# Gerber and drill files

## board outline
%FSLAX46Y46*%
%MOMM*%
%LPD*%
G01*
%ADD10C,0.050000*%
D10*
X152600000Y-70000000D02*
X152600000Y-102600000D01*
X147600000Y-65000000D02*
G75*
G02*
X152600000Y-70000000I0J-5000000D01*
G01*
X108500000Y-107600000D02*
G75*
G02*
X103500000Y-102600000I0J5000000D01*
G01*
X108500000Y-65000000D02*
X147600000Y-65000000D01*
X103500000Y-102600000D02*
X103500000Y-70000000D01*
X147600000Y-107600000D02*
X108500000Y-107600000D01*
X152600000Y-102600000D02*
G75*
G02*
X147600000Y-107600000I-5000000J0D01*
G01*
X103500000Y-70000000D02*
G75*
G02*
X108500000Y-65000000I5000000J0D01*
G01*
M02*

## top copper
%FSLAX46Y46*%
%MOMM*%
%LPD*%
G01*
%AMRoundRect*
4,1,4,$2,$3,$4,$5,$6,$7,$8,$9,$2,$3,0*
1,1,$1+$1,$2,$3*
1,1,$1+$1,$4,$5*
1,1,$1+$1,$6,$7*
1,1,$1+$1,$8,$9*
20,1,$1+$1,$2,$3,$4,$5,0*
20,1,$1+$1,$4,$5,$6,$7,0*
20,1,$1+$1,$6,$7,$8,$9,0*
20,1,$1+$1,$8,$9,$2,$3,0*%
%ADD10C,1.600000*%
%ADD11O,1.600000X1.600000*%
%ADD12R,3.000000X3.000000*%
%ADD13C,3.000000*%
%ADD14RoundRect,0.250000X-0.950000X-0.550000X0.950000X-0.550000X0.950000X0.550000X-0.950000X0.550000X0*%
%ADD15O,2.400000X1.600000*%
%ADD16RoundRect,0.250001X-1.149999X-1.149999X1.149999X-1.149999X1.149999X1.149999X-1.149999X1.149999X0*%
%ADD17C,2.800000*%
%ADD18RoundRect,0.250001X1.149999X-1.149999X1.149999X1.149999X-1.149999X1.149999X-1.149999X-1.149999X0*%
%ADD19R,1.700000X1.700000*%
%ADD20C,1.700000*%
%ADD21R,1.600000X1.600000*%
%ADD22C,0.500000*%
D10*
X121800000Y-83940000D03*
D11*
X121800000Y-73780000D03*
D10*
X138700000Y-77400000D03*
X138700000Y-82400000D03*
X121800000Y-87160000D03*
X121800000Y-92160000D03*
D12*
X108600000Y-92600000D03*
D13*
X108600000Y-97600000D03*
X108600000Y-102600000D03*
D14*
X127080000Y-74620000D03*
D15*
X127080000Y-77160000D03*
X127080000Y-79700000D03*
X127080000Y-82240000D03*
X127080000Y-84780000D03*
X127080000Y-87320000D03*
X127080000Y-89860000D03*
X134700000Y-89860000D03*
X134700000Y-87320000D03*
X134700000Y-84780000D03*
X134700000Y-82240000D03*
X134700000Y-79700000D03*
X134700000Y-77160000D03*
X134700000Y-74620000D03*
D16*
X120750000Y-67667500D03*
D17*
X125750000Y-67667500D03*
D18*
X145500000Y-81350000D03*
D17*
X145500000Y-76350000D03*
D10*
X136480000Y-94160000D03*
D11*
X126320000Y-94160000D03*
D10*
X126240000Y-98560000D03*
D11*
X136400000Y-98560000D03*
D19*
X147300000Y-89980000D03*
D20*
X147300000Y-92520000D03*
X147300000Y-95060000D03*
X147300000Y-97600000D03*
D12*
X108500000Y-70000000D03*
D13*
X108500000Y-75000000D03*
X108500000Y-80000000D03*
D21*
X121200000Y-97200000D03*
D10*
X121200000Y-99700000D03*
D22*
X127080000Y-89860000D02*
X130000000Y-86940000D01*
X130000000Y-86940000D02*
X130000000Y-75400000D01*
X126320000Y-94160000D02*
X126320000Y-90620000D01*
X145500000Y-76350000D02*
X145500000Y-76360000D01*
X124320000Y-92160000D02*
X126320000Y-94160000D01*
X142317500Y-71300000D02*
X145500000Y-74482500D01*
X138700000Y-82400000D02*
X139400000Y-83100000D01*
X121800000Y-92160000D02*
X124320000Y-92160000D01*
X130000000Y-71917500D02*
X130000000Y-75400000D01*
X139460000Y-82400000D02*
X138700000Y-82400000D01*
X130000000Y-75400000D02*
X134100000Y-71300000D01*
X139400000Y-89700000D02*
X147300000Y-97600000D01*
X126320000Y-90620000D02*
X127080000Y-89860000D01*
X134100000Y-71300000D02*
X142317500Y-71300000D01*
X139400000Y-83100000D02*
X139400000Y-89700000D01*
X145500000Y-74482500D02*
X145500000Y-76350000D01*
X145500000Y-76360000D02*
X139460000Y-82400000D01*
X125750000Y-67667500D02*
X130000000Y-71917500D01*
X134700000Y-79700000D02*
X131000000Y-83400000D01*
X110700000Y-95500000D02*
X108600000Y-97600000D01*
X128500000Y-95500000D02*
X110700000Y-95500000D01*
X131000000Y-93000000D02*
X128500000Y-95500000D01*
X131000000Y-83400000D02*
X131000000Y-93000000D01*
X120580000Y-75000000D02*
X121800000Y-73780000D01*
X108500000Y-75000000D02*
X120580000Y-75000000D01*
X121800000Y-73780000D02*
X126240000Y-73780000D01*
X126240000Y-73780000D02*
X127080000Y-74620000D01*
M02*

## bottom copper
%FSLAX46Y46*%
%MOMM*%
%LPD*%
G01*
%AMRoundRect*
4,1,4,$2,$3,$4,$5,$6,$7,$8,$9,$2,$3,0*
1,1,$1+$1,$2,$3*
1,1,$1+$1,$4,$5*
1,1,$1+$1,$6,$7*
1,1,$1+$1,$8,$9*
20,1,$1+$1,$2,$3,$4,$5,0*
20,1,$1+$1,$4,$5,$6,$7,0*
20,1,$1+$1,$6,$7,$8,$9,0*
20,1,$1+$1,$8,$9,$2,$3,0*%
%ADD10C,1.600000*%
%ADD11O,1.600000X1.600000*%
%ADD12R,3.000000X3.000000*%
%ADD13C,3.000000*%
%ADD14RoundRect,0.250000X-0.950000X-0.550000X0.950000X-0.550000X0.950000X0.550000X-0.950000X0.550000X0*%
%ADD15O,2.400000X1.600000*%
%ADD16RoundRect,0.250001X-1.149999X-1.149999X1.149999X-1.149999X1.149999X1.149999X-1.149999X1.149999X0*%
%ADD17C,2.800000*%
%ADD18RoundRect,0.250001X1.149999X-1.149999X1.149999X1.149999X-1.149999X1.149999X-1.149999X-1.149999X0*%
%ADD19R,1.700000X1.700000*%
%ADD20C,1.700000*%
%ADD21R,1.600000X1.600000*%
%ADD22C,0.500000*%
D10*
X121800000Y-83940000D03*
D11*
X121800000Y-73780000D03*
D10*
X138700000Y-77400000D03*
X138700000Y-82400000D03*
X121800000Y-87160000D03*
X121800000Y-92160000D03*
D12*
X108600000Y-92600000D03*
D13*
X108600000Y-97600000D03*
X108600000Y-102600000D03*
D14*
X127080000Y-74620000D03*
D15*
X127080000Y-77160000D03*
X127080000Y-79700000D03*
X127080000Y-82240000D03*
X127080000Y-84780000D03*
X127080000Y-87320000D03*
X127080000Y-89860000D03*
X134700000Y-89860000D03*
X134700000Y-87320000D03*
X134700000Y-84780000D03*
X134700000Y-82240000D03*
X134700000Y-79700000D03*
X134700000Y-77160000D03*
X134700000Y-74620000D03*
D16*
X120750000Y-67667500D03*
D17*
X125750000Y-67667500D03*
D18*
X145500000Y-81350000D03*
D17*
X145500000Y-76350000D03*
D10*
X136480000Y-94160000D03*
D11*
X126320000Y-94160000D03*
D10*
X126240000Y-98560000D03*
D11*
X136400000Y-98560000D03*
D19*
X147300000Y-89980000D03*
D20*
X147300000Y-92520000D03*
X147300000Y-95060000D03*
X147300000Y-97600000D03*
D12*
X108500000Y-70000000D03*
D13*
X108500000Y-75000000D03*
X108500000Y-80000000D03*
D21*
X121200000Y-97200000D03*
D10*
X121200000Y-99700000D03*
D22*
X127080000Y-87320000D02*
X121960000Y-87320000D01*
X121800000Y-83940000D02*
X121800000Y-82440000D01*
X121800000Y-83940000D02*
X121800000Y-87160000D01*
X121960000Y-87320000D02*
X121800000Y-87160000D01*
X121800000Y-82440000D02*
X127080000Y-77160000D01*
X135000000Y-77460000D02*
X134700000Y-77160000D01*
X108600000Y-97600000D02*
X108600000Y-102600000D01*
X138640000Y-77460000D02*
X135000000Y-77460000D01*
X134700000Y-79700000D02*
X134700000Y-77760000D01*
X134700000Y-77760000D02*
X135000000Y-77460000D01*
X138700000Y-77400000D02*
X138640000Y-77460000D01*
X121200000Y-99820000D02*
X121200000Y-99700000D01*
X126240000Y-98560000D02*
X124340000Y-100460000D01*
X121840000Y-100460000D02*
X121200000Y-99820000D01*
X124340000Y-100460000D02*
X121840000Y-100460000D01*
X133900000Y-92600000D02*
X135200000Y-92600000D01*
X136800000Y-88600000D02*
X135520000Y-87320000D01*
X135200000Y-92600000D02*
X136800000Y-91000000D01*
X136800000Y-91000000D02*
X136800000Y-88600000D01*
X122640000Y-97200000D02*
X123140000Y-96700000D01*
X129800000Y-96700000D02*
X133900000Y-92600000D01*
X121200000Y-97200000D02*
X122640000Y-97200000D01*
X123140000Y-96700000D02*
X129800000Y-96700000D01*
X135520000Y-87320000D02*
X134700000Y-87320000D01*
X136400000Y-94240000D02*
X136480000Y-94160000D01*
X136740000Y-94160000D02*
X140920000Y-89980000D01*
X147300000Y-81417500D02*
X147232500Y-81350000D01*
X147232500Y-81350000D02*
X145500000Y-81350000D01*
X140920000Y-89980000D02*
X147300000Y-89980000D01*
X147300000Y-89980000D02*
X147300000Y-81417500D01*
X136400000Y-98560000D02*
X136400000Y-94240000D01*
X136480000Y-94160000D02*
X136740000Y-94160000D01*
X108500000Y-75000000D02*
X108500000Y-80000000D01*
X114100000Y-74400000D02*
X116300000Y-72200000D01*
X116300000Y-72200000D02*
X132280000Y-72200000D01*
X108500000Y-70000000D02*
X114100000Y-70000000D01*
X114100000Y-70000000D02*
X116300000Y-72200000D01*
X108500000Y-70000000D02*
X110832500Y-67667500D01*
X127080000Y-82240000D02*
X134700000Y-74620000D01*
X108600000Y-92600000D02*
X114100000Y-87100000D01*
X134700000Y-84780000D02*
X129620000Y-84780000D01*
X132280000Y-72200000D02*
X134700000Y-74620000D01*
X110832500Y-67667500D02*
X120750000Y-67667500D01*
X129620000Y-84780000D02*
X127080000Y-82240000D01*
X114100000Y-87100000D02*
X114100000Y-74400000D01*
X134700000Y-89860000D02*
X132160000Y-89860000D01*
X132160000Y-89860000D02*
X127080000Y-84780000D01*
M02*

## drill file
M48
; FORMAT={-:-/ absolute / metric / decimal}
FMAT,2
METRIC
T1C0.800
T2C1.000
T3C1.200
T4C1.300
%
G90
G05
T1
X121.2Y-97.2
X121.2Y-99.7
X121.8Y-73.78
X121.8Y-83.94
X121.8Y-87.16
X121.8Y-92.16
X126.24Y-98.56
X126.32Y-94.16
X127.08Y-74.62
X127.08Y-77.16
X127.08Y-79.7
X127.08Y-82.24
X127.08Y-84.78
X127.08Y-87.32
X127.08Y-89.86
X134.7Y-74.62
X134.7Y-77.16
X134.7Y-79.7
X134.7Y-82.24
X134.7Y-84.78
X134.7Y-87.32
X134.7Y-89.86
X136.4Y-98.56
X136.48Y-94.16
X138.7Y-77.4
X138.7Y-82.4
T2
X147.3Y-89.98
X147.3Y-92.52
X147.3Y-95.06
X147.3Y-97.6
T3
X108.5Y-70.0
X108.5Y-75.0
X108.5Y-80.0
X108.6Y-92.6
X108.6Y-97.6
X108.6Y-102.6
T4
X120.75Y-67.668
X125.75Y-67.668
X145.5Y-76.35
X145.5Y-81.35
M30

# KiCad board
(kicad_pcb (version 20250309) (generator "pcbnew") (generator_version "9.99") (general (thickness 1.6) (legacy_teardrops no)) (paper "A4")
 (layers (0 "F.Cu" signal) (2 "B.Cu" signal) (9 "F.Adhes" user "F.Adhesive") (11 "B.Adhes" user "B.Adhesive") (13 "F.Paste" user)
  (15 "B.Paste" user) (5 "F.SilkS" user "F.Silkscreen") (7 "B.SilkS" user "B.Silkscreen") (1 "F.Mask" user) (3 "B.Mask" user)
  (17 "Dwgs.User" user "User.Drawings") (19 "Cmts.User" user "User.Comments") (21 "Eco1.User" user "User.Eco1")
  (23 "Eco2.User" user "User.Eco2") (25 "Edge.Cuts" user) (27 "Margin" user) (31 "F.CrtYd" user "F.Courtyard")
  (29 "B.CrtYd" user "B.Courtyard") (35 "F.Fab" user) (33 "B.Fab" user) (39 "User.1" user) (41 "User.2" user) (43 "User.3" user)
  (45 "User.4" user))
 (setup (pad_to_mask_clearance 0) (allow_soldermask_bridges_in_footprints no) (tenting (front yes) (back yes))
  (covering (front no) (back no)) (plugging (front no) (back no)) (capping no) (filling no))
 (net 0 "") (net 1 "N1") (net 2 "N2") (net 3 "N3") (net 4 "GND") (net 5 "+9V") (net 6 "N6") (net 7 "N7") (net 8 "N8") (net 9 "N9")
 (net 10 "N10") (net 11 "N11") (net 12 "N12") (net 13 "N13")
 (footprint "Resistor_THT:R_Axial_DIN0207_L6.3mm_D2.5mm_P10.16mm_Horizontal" (layer "F.Cu") (at 121.8 83.94 90)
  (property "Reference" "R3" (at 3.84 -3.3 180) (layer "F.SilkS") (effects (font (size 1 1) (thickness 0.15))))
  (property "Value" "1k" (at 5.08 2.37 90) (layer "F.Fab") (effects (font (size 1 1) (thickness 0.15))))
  (pad "1" thru_hole circle (at 0 0 90) (size 1.6 1.6) (drill 0.8) (layers "*.Cu" "*.Mask") (remove_unused_layers no) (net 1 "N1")
   (tenting (front none) (back none)))
  (pad "2" thru_hole oval (at 10.16 0 90) (size 1.6 1.6) (drill 0.8) (layers "*.Cu" "*.Mask") (remove_unused_layers no) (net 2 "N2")
   (tenting (front none) (back none))))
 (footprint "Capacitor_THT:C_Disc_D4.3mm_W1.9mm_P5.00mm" (layer "F.Cu") (at 138.7 77.4 -90)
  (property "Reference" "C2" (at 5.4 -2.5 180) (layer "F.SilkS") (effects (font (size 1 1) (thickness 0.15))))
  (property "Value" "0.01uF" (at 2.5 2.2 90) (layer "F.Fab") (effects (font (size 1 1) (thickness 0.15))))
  (pad "1" thru_hole circle (at 0 0 270) (size 1.6 1.6) (drill 0.8) (layers "*.Cu" "*.Mask") (remove_unused_layers no) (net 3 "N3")
   (tenting (front none) (back none)))
  (pad "2" thru_hole circle (at 5 0 270) (size 1.6 1.6) (drill 0.8) (layers "*.Cu" "*.Mask") (remove_unused_layers no) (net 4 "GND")
   (tenting (front none) (back none))))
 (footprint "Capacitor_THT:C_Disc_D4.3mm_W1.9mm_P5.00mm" (layer "F.Cu") (at 121.8 87.16 -90)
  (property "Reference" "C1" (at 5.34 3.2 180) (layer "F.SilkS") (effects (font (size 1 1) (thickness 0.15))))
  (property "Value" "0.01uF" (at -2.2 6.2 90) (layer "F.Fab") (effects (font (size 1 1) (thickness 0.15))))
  (pad "1" thru_hole circle (at 0 0 270) (size 1.6 1.6) (drill 0.8) (layers "*.Cu" "*.Mask") (remove_unused_layers no) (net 1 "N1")
   (tenting (front none) (back none)))
  (pad "2" thru_hole circle (at 5 0 270) (size 1.6 1.6) (drill 0.8) (layers "*.Cu" "*.Mask") (remove_unused_layers no) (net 4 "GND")
   (tenting (front none) (back none))))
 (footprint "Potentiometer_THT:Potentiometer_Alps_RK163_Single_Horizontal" (layer "F.Cu") (at 108.6 92.6)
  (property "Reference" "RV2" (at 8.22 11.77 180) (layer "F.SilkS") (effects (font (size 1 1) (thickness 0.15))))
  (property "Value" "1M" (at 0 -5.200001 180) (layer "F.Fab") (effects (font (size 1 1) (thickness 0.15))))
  (pad "1" thru_hole rect (at 0 0 180) (size 3 3) (drill 1.2) (layers "*.Cu" "*.Mask") (remove_unused_layers no) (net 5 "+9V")
   (tenting (front none) (back none)))
  (pad "2" thru_hole circle (at 0 5 180) (size 3 3) (drill 1.2) (layers "*.Cu" "*.Mask") (remove_unused_layers no) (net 3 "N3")
   (tenting (front none) (back none)))
  (pad "3" thru_hole circle (at 0 10 180) (size 3 3) (drill 1.2) (layers "*.Cu" "*.Mask") (remove_unused_layers no) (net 3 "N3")
   (tenting (front none) (back none))))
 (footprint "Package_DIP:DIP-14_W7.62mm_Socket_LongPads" (layer "F.Cu") (at 127.08 74.62)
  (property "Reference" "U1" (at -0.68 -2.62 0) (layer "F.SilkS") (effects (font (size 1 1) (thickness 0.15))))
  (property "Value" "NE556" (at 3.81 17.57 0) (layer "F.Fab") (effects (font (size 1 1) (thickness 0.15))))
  (pad "1" thru_hole roundrect (at 0 0) (size 2.4 1.6) (drill 0.8) (layers "*.Cu" "*.Mask") (remove_unused_layers no)
   (roundrect_rratio 0.15625) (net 2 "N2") (tenting (front none) (back none)))
  (pad "2" thru_hole oval (at 0 2.54) (size 2.4 1.6) (drill 0.8) (layers "*.Cu" "*.Mask") (remove_unused_layers no) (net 1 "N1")
   (tenting (front none) (back none)))
  (pad "3" thru_hole oval (at 0 5.08) (size 2.4 1.6) (drill 0.8) (layers "*.Cu" "*.Mask") (remove_unused_layers no) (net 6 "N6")
   (tenting (front none) (back none)))
  (pad "4" thru_hole oval (at 0 7.62) (size 2.4 1.6) (drill 0.8) (layers "*.Cu" "*.Mask") (remove_unused_layers no) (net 5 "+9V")
   (tenting (front none) (back none)))
  (pad "5" thru_hole oval (at 0 10.16) (size 2.4 1.6) (drill 0.8) (layers "*.Cu" "*.Mask") (remove_unused_layers no) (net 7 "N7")
   (tenting (front none) (back none)))
  (pad "6" thru_hole oval (at 0 12.7) (size 2.4 1.6) (drill 0.8) (layers "*.Cu" "*.Mask") (remove_unused_layers no) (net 1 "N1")
   (tenting (front none) (back none)))
  (pad "7" thru_hole oval (at 0 15.24) (size 2.4 1.6) (drill 0.8) (layers "*.Cu" "*.Mask") (remove_unused_layers no) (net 4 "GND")
   (tenting (front none) (back none)))
  (pad "8" thru_hole oval (at 7.62 15.24) (size 2.4 1.6) (drill 0.8) (layers "*.Cu" "*.Mask") (remove_unused_layers no) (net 7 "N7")
   (tenting (front none) (back none)))
  (pad "9" thru_hole oval (at 7.62 12.7) (size 2.4 1.6) (drill 0.8) (layers "*.Cu" "*.Mask") (remove_unused_layers no) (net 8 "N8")
   (tenting (front none) (back none)))
  (pad "10" thru_hole oval (at 7.62 10.16) (size 2.4 1.6) (drill 0.8) (layers "*.Cu" "*.Mask") (remove_unused_layers no) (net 5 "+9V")
   (tenting (front none) (back none)))
  (pad "11" thru_hole oval (at 7.62 7.62) (size 2.4 1.6) (drill 0.8) (layers "*.Cu" "*.Mask") (remove_unused_layers no) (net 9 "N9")
   (tenting (front none) (back none)))
  (pad "12" thru_hole oval (at 7.62 5.08) (size 2.4 1.6) (drill 0.8) (layers "*.Cu" "*.Mask") (remove_unused_layers no) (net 3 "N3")
   (tenting (front none) (back none)))
  (pad "13" thru_hole oval (at 7.62 2.54) (size 2.4 1.6) (drill 0.8) (layers "*.Cu" "*.Mask") (remove_unused_layers no) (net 3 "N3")
   (tenting (front none) (back none)))
  (pad "14" thru_hole oval (at 7.62 0) (size 2.4 1.6) (drill 0.8) (layers "*.Cu" "*.Mask") (remove_unused_layers no) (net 5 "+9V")
   (tenting (front none) (back none))))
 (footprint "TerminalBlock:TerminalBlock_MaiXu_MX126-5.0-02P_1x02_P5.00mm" (layer "F.Cu") (at 120.75 67.6675)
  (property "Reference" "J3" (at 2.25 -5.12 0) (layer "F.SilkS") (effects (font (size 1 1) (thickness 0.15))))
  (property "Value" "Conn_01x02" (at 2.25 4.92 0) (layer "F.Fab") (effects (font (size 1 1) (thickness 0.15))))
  (pad "1" thru_hole roundrect (at 0 0) (size 2.8 2.8) (drill 1.3) (layers "*.Cu" "*.Mask") (remove_unused_layers no)
   (roundrect_rratio 0.089286) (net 5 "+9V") (tenting (front none) (back none)))
  (pad "2" thru_hole circle (at 5 0) (size 2.8 2.8) (drill 1.3) (layers "*.Cu" "*.Mask") (remove_unused_layers no) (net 4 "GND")
   (tenting (front none) (back none))))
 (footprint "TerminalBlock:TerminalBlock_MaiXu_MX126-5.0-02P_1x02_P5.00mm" (layer "F.Cu") (at 145.5 81.35 90)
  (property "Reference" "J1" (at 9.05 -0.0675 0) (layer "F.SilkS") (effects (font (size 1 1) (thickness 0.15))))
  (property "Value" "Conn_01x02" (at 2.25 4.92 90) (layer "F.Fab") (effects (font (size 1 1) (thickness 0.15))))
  (pad "1" thru_hole roundrect (at 0 0 90) (size 2.8 2.8) (drill 1.3) (layers "*.Cu" "*.Mask") (remove_unused_layers no)
   (roundrect_rratio 0.089286) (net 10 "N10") (tenting (front none) (back none)))
  (pad "2" thru_hole circle (at 5 0 90) (size 2.8 2.8) (drill 1.3) (layers "*.Cu" "*.Mask") (remove_unused_layers no) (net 4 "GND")
   (tenting (front none) (back none))))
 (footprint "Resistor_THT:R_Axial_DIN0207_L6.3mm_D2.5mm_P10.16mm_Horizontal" (layer "F.Cu") (at 136.48 94.16 180)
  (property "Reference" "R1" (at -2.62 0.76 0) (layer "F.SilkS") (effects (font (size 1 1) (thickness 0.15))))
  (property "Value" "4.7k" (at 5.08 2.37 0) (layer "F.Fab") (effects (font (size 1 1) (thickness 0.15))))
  (pad "1" thru_hole circle (at 0 0 180) (size 1.6 1.6) (drill 0.8) (layers "*.Cu" "*.Mask") (remove_unused_layers no) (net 10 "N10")
   (tenting (front none) (back none)))
  (pad "2" thru_hole oval (at 10.16 0 180) (size 1.6 1.6) (drill 0.8) (layers "*.Cu" "*.Mask") (remove_unused_layers no) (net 4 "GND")
   (tenting (front none) (back none))))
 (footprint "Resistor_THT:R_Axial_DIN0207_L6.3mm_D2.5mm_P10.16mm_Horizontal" (layer "F.Cu") (at 126.24 98.56)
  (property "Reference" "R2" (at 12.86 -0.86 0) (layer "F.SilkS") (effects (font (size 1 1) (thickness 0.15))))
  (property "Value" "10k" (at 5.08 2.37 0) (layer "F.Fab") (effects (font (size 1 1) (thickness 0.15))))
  (pad "1" thru_hole circle (at 0 0) (size 1.6 1.6) (drill 0.8) (layers "*.Cu" "*.Mask") (remove_unused_layers no) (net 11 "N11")
   (tenting (front none) (back none)))
  (pad "2" thru_hole oval (at 10.16 0) (size 1.6 1.6) (drill 0.8) (layers "*.Cu" "*.Mask") (remove_unused_layers no) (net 10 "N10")
   (tenting (front none) (back none))))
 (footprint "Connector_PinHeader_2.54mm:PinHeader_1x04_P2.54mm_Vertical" (layer "F.Cu") (at 147.3 89.98)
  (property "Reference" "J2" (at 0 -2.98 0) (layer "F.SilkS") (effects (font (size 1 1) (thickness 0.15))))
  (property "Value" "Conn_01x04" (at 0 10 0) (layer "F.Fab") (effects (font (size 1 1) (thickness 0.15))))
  (pad "1" thru_hole rect (at 0 0) (size 1.7 1.7) (drill 1) (layers "*.Cu" "*.Mask") (remove_unused_layers no) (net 10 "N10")
   (tenting (front none) (back none)))
  (pad "2" thru_hole circle (at 0 2.54) (size 1.7 1.7) (drill 1) (layers "*.Cu" "*.Mask") (remove_unused_layers no) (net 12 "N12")
   (tenting (front none) (back none)))
  (pad "3" thru_hole circle (at 0 5.08) (size 1.7 1.7) (drill 1) (layers "*.Cu" "*.Mask") (remove_unused_layers no) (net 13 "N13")
   (tenting (front none) (back none)))
  (pad "4" thru_hole circle (at 0 7.62) (size 1.7 1.7) (drill 1) (layers "*.Cu" "*.Mask") (remove_unused_layers no) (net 4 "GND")
   (tenting (front none) (back none))))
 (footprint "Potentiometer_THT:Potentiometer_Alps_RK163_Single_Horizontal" (layer "F.Cu") (at 108.5 70)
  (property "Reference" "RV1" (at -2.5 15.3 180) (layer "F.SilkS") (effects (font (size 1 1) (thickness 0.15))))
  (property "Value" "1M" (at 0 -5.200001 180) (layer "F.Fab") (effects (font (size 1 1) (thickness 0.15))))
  (pad "1" thru_hole rect (at 0 0 180) (size 3 3) (drill 1.2) (layers "*.Cu" "*.Mask") (remove_unused_layers no) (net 5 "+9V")
   (tenting (front none) (back none)))
  (pad "2" thru_hole circle (at 0 5 180) (size 3 3) (drill 1.2) (layers "*.Cu" "*.Mask") (remove_unused_layers no) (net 2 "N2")
   (tenting (front none) (back none)))
  (pad "3" thru_hole circle (at 0 10 180) (size 3 3) (drill 1.2) (layers "*.Cu" "*.Mask") (remove_unused_layers no) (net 2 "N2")
   (tenting (front none) (back none))))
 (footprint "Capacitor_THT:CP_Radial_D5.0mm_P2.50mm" (layer "F.Cu") (at 121.2 97.2 -90)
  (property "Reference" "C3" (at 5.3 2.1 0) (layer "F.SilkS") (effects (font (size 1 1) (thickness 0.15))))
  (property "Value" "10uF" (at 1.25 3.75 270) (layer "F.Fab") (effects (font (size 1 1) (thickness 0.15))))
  (pad "1" thru_hole rect (at 0 0 270) (size 1.6 1.6) (drill 0.8) (layers "*.Cu" "*.Mask") (remove_unused_layers no) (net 8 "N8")
   (tenting (front none) (back none)))
  (pad "2" thru_hole circle (at 2.5 0 270) (size 1.6 1.6) (drill 0.8) (layers "*.Cu" "*.Mask") (remove_unused_layers no) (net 11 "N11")
   (tenting (front none) (back none))))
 (gr_line (start 152.6 70) (end 152.6 102.6) (stroke (width 0.05) (type default)) (layer "Edge.Cuts"))
 (gr_arc (start 147.6 65) (mid 151.135534 66.464466) (end 152.6 70) (stroke (width 0.05) (type default)) (layer "Edge.Cuts"))
 (gr_arc (start 108.5 107.6) (mid 104.964466 106.135534) (end 103.5 102.6) (stroke (width 0.05) (type default)) (layer "Edge.Cuts"))
 (gr_line (start 108.5 65) (end 147.6 65) (stroke (width 0.05) (type default)) (layer "Edge.Cuts"))
 (gr_line (start 103.5 102.6) (end 103.5 70) (stroke (width 0.05) (type default)) (layer "Edge.Cuts"))
 (gr_line (start 147.6 107.6) (end 108.5 107.6) (stroke (width 0.05) (type default)) (layer "Edge.Cuts"))
 (gr_arc (start 152.6 102.6) (mid 151.135534 106.135534) (end 147.6 107.6) (stroke (width 0.05) (type default)) (layer "Edge.Cuts"))
 (gr_arc (start 103.5 70) (mid 104.964466 66.464466) (end 108.5 65) (stroke (width 0.05) (type default)) (layer "Edge.Cuts"))
 (segment (start 127.08 89.86) (end 130 86.94) (width 0.5) (layer "F.Cu") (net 4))
 (segment (start 130 86.94) (end 130 75.4) (width 0.5) (layer "F.Cu") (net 4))
 (segment (start 126.32 94.16) (end 126.32 90.62) (width 0.5) (layer "F.Cu") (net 4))
 (segment (start 145.5 76.35) (end 145.5 76.36) (width 0.5) (layer "F.Cu") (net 4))
 (segment (start 124.32 92.16) (end 126.32 94.16) (width 0.5) (layer "F.Cu") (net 4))
 (segment (start 142.3175 71.3) (end 145.5 74.4825) (width 0.5) (layer "F.Cu") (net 4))
 (segment (start 138.7 82.4) (end 139.4 83.1) (width 0.5) (layer "F.Cu") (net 4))
 (segment (start 121.8 92.16) (end 124.32 92.16) (width 0.5) (layer "F.Cu") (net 4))
 (segment (start 130 71.9175) (end 130 75.4) (width 0.5) (layer "F.Cu") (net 4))
 (segment (start 139.46 82.4) (end 138.7 82.4) (width 0.5) (layer "F.Cu") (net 4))
 (segment (start 130 75.4) (end 134.1 71.3) (width 0.5) (layer "F.Cu") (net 4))
 (segment (start 139.4 89.7) (end 147.3 97.6) (width 0.5) (layer "F.Cu") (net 4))
 (segment (start 126.32 90.62) (end 127.08 89.86) (width 0.5) (layer "F.Cu") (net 4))
 (segment (start 134.1 71.3) (end 142.3175 71.3) (width 0.5) (layer "F.Cu") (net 4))
 (segment (start 139.4 83.1) (end 139.4 89.7) (width 0.5) (layer "F.Cu") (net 4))
 (segment (start 145.5 74.4825) (end 145.5 76.35) (width 0.5) (layer "F.Cu") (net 4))
 (segment (start 145.5 76.36) (end 139.46 82.4) (width 0.5) (layer "F.Cu") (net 4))
 (segment (start 125.75 67.6675) (end 130 71.9175) (width 0.5) (layer "F.Cu") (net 4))
 (segment (start 127.08 87.32) (end 121.96 87.32) (width 0.5) (layer "B.Cu") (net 1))
 (segment (start 121.8 83.94) (end 121.8 82.44) (width 0.5) (layer "B.Cu") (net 1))
 (segment (start 121.8 83.94) (end 121.8 87.16) (width 0.5) (layer "B.Cu") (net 1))
 (segment (start 121.96 87.32) (end 121.8 87.16) (width 0.5) (layer "B.Cu") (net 1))
 (segment (start 121.8 82.44) (end 127.08 77.16) (width 0.5) (layer "B.Cu") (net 1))
 (segment (start 134.7 79.7) (end 131 83.4) (width 0.5) (layer "F.Cu") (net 3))
 (segment (start 110.7 95.5) (end 108.6 97.6) (width 0.5) (layer "F.Cu") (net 3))
 (segment (start 128.5 95.5) (end 110.7 95.5) (width 0.5) (layer "F.Cu") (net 3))
 (segment (start 131 93) (end 128.5 95.5) (width 0.5) (layer "F.Cu") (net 3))
 (segment (start 131 83.4) (end 131 93) (width 0.5) (layer "F.Cu") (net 3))
 (segment (start 135 77.46) (end 134.7 77.16) (width 0.5) (layer "B.Cu") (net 3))
 (segment (start 108.6 97.6) (end 108.6 102.6) (width 0.5) (layer "B.Cu") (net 3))
 (segment (start 138.64 77.46) (end 135 77.46) (width 0.5) (layer "B.Cu") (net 3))
 (segment (start 134.7 79.7) (end 134.7 77.76) (width 0.5) (layer "B.Cu") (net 3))
 (segment (start 134.7 77.76) (end 135 77.46) (width 0.5) (layer "B.Cu") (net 3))
 (segment (start 138.7 77.4) (end 138.64 77.46) (width 0.5) (layer "B.Cu") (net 3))
 (segment (start 121.2 99.82) (end 121.2 99.7) (width 0.5) (layer "B.Cu") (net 11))
 (segment (start 126.24 98.56) (end 124.34 100.46) (width 0.5) (layer "B.Cu") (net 11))
 (segment (start 121.84 100.46) (end 121.2 99.82) (width 0.5) (layer "B.Cu") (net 11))
 (segment (start 124.34 100.46) (end 121.84 100.46) (width 0.5) (layer "B.Cu") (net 11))
 (segment (start 133.9 92.6) (end 135.2 92.6) (width 0.5) (layer "B.Cu") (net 8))
 (segment (start 136.8 88.6) (end 135.52 87.32) (width 0.5) (layer "B.Cu") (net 8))
 (segment (start 135.2 92.6) (end 136.8 91) (width 0.5) (layer "B.Cu") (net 8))
 (segment (start 136.8 91) (end 136.8 88.6) (width 0.5) (layer "B.Cu") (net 8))
 (segment (start 122.64 97.2) (end 123.14 96.7) (width 0.5) (layer "B.Cu") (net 8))
 (segment (start 129.8 96.7) (end 133.9 92.6) (width 0.5) (layer "B.Cu") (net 8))
 (segment (start 121.2 97.2) (end 122.64 97.2) (width 0.5) (layer "B.Cu") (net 8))
 (segment (start 123.14 96.7) (end 129.8 96.7) (width 0.5) (layer "B.Cu") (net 8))
 (segment (start 135.52 87.32) (end 134.7 87.32) (width 0.5) (layer "B.Cu") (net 8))
 (segment (start 136.4 94.24) (end 136.48 94.16) (width 0.5) (layer "B.Cu") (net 10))
 (segment (start 136.74 94.16) (end 140.92 89.98) (width 0.5) (layer "B.Cu") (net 10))
 (segment (start 147.3 81.4175) (end 147.2325 81.35) (width 0.5) (layer "B.Cu") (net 10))
 (segment (start 147.2325 81.35) (end 145.5 81.35) (width 0.5) (layer "B.Cu") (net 10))
 (segment (start 140.92 89.98) (end 147.3 89.98) (width 0.5) (layer "B.Cu") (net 10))
 (segment (start 147.3 89.98) (end 147.3 81.4175) (width 0.5) (layer "B.Cu") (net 10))
 (segment (start 136.4 98.56) (end 136.4 94.24) (width 0.5) (layer "B.Cu") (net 10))
 (segment (start 136.48 94.16) (end 136.74 94.16) (width 0.5) (layer "B.Cu") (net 10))
 (segment (start 120.58 75) (end 121.8 73.78) (width 0.5) (layer "F.Cu") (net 2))
 (segment (start 108.5 75) (end 120.58 75) (width 0.5) (layer "F.Cu") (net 2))
 (segment (start 121.8 73.78) (end 126.24 73.78) (width 0.5) (layer "F.Cu") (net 2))
 (segment (start 126.24 73.78) (end 127.08 74.62) (width 0.5) (layer "F.Cu") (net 2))
 (segment (start 108.5 75) (end 108.5 80) (width 0.5) (layer "B.Cu") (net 2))
 (segment (start 114.1 74.4) (end 116.3 72.2) (width 0.5) (layer "B.Cu") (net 5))
 (segment (start 116.3 72.2) (end 132.28 72.2) (width 0.5) (layer "B.Cu") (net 5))
 (segment (start 108.5 70) (end 114.1 70) (width 0.5) (layer "B.Cu") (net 5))
 (segment (start 114.1 70) (end 116.3 72.2) (width 0.5) (layer "B.Cu") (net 5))
 (segment (start 108.5 70) (end 110.8325 67.6675) (width 0.5) (layer "B.Cu") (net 5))
 (segment (start 127.08 82.24) (end 134.7 74.62) (width 0.5) (layer "B.Cu") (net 5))
 (segment (start 108.6 92.6) (end 114.1 87.1) (width 0.5) (layer "B.Cu") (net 5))
 (segment (start 134.7 84.78) (end 129.62 84.78) (width 0.5) (layer "B.Cu") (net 5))
 (segment (start 132.28 72.2) (end 134.7 74.62) (width 0.5) (layer "B.Cu") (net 5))
 (segment (start 110.8325 67.6675) (end 120.75 67.6675) (width 0.5) (layer "B.Cu") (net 5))
 (segment (start 129.62 84.78) (end 127.08 82.24) (width 0.5) (layer "B.Cu") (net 5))
 (segment (start 114.1 87.1) (end 114.1 74.4) (width 0.5) (layer "B.Cu") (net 5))
 (segment (start 134.7 89.86) (end 132.16 89.86) (width 0.5) (layer "B.Cu") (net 7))
 (segment (start 132.16 89.86) (end 127.08 84.78) (width 0.5) (layer "B.Cu") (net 7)))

